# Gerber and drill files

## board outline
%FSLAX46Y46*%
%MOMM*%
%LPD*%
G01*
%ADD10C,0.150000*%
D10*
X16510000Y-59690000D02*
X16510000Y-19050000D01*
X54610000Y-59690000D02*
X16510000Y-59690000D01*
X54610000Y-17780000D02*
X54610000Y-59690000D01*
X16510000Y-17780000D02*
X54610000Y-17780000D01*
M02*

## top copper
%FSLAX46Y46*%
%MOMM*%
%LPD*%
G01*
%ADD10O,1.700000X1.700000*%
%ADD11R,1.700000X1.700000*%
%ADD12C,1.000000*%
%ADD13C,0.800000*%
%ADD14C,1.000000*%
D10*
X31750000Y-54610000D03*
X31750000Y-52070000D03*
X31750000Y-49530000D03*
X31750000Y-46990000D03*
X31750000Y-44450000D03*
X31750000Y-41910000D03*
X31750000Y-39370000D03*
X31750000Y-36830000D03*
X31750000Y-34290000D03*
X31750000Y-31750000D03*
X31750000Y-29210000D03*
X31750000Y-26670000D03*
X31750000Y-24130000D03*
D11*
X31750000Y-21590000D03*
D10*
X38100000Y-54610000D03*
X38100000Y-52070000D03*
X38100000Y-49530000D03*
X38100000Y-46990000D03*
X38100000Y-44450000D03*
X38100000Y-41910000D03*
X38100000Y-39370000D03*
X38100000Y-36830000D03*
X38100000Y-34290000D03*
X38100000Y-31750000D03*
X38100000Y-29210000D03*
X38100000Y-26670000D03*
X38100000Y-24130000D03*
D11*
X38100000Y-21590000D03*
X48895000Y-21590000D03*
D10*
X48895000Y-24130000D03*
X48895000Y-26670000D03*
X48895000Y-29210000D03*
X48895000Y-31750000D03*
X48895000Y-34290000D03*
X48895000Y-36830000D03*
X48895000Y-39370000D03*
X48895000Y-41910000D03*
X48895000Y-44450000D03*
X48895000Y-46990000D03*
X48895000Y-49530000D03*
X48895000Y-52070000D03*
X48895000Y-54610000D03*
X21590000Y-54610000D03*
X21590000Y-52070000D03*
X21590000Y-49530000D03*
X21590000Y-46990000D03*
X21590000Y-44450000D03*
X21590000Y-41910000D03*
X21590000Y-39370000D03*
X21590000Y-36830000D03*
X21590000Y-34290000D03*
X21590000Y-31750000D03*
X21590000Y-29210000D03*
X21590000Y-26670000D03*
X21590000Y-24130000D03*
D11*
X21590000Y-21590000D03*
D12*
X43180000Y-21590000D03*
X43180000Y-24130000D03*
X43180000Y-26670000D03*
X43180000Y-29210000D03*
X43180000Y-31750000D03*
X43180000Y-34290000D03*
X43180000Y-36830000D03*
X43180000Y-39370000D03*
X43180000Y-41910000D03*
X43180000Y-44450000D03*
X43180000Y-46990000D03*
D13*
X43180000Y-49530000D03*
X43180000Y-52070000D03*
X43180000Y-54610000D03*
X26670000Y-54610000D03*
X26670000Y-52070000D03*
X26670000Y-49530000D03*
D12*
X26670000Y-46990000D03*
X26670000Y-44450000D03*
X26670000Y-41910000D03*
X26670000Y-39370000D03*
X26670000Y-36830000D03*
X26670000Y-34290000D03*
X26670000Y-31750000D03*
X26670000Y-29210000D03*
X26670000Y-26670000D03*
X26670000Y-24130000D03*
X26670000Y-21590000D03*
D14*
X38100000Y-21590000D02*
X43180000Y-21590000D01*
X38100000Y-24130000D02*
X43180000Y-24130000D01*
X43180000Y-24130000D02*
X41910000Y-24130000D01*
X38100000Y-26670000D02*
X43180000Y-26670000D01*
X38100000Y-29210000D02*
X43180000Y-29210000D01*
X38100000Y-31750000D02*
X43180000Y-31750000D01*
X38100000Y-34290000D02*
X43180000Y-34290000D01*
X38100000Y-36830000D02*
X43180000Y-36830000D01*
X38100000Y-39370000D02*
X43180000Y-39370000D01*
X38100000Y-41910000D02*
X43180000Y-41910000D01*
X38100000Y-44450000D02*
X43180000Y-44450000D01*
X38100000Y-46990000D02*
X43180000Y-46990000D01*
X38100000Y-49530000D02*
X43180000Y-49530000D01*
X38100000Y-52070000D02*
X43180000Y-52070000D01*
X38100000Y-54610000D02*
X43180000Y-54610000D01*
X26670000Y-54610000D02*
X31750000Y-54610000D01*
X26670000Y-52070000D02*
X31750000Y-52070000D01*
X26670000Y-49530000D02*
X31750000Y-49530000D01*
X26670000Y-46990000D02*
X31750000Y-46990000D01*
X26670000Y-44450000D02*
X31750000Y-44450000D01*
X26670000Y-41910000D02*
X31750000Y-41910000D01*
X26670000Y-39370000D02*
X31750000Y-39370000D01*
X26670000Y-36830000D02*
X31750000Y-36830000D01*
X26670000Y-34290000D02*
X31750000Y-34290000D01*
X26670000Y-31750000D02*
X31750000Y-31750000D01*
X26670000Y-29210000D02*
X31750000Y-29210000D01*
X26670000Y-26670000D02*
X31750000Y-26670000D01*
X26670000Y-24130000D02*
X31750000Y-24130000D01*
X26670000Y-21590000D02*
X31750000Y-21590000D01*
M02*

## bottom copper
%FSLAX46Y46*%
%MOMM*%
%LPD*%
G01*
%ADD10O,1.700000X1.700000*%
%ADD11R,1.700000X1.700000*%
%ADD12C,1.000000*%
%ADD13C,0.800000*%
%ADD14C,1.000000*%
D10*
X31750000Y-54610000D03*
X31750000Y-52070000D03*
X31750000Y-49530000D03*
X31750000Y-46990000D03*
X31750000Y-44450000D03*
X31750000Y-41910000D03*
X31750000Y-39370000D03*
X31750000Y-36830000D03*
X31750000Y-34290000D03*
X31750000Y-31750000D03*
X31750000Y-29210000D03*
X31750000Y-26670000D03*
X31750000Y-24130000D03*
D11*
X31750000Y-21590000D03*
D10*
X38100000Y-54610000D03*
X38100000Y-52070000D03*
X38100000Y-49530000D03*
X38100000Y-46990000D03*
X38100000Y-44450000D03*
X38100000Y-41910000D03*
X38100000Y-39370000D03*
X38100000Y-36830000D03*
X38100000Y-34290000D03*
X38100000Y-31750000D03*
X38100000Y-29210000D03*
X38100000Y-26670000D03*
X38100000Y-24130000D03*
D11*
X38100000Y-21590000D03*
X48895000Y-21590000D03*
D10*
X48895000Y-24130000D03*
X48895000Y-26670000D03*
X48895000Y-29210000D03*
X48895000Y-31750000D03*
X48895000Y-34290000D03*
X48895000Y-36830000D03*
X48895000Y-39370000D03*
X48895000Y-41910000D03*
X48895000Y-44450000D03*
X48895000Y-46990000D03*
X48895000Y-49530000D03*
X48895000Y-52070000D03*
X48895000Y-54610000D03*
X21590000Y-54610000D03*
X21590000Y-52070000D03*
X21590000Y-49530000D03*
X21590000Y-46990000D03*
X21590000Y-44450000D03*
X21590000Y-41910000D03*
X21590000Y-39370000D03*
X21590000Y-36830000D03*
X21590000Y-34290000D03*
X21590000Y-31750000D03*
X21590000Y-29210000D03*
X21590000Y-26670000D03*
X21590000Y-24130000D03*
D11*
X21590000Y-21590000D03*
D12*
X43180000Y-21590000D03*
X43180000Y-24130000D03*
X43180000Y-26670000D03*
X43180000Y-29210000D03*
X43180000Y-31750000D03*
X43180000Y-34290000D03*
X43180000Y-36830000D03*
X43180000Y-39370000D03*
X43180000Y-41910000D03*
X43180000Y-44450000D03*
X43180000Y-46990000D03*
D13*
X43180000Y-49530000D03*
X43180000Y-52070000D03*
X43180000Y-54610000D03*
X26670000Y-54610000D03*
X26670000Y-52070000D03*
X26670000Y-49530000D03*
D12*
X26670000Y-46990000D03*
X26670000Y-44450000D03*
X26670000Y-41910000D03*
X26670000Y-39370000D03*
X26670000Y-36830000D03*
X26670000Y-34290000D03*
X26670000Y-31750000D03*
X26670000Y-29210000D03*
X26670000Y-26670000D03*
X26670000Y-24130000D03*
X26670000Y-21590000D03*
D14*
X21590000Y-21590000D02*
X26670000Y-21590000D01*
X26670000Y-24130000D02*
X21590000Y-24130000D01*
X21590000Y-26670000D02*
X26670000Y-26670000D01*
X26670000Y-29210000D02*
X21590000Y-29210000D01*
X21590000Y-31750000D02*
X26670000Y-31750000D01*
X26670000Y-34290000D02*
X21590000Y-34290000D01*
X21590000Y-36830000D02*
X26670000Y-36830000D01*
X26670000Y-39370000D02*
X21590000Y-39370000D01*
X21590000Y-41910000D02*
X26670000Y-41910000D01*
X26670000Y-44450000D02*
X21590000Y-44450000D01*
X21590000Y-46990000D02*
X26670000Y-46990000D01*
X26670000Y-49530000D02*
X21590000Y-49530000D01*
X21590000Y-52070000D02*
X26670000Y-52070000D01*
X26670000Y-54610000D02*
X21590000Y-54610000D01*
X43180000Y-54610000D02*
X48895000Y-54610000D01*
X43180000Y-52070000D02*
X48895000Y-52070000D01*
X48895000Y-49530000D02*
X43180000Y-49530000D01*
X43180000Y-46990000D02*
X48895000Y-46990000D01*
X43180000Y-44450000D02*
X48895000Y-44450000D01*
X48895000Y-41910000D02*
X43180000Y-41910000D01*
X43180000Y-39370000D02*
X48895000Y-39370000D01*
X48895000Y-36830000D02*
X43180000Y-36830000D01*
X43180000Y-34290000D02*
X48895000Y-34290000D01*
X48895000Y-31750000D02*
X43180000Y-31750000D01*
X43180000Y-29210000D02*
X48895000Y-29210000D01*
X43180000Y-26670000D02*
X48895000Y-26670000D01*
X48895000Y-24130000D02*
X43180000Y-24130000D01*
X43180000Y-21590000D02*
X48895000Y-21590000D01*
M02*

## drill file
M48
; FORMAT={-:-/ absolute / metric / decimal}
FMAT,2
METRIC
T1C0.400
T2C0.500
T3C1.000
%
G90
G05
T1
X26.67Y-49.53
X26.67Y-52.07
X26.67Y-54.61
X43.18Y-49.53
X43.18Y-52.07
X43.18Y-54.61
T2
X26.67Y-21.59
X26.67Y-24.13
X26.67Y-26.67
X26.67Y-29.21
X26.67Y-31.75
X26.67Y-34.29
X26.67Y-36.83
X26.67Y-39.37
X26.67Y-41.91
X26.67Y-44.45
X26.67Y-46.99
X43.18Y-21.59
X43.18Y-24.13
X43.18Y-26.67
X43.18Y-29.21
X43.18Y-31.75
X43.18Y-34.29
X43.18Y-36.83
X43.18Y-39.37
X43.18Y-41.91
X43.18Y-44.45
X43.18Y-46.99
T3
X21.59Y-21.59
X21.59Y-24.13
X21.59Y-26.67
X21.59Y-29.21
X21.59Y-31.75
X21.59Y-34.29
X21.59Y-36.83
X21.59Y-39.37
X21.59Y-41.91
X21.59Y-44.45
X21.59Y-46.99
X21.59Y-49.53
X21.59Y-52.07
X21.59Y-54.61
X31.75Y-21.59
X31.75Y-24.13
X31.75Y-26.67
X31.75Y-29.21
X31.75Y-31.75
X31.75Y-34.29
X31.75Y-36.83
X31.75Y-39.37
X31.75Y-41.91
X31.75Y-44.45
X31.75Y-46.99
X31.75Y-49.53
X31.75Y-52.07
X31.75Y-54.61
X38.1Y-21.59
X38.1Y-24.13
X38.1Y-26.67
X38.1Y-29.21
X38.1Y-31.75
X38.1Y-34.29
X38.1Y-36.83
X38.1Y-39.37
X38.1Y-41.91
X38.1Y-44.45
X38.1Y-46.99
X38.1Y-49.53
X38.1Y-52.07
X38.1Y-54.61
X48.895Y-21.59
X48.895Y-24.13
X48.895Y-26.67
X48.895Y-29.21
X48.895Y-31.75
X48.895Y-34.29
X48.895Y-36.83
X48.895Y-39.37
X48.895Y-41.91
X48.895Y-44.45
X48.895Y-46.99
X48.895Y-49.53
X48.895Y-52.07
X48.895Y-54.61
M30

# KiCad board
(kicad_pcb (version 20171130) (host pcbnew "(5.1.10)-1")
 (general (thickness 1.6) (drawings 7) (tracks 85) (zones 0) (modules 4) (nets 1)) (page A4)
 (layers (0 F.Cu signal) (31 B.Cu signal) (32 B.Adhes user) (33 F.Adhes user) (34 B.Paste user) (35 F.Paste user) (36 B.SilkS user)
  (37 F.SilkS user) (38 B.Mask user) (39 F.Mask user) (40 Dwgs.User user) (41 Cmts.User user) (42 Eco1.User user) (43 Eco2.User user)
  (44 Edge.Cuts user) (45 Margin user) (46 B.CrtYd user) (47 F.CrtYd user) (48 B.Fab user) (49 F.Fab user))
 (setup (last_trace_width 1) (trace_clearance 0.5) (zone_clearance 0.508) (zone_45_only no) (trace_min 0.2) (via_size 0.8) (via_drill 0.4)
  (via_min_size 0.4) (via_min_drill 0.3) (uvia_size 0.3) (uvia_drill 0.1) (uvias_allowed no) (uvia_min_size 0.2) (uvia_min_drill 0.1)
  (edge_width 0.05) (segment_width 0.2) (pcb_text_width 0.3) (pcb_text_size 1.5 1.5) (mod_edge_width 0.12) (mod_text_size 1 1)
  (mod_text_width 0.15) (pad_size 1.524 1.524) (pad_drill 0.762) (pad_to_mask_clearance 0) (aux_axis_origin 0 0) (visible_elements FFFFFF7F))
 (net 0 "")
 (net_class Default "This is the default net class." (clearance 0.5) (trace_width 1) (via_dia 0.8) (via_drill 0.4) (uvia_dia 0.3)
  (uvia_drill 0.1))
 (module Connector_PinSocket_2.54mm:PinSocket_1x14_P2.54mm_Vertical (layer F.Cu) (at 31.75 21.59)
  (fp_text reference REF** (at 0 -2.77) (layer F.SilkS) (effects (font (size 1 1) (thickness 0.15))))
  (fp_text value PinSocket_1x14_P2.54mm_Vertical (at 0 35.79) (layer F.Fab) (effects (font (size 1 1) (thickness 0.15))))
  (pad 14 thru_hole oval (at 0 33.02) (size 1.7 1.7) (drill 1) (layers *.Cu *.Mask))
  (pad 13 thru_hole oval (at 0 30.48) (size 1.7 1.7) (drill 1) (layers *.Cu *.Mask))
  (pad 12 thru_hole oval (at 0 27.94) (size 1.7 1.7) (drill 1) (layers *.Cu *.Mask))
  (pad 11 thru_hole oval (at 0 25.4) (size 1.7 1.7) (drill 1) (layers *.Cu *.Mask))
  (pad 10 thru_hole oval (at 0 22.86) (size 1.7 1.7) (drill 1) (layers *.Cu *.Mask))
  (pad 9 thru_hole oval (at 0 20.32) (size 1.7 1.7) (drill 1) (layers *.Cu *.Mask))
  (pad 8 thru_hole oval (at 0 17.78) (size 1.7 1.7) (drill 1) (layers *.Cu *.Mask))
  (pad 7 thru_hole oval (at 0 15.24) (size 1.7 1.7) (drill 1) (layers *.Cu *.Mask))
  (pad 6 thru_hole oval (at 0 12.7) (size 1.7 1.7) (drill 1) (layers *.Cu *.Mask))
  (pad 5 thru_hole oval (at 0 10.16) (size 1.7 1.7) (drill 1) (layers *.Cu *.Mask))
  (pad 4 thru_hole oval (at 0 7.62) (size 1.7 1.7) (drill 1) (layers *.Cu *.Mask))
  (pad 3 thru_hole oval (at 0 5.08) (size 1.7 1.7) (drill 1) (layers *.Cu *.Mask))
  (pad 2 thru_hole oval (at 0 2.54) (size 1.7 1.7) (drill 1) (layers *.Cu *.Mask))
  (pad 1 thru_hole rect (at 0 0) (size 1.7 1.7) (drill 1) (layers *.Cu *.Mask)))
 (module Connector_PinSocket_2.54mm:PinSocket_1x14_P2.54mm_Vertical (layer F.Cu) (at 38.1 21.59)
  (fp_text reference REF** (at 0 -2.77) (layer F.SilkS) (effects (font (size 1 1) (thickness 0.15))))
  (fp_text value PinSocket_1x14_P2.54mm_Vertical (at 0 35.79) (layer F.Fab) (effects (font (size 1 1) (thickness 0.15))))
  (pad 14 thru_hole oval (at 0 33.02) (size 1.7 1.7) (drill 1) (layers *.Cu *.Mask))
  (pad 13 thru_hole oval (at 0 30.48) (size 1.7 1.7) (drill 1) (layers *.Cu *.Mask))
  (pad 12 thru_hole oval (at 0 27.94) (size 1.7 1.7) (drill 1) (layers *.Cu *.Mask))
  (pad 11 thru_hole oval (at 0 25.4) (size 1.7 1.7) (drill 1) (layers *.Cu *.Mask))
  (pad 10 thru_hole oval (at 0 22.86) (size 1.7 1.7) (drill 1) (layers *.Cu *.Mask))
  (pad 9 thru_hole oval (at 0 20.32) (size 1.7 1.7) (drill 1) (layers *.Cu *.Mask))
  (pad 8 thru_hole oval (at 0 17.78) (size 1.7 1.7) (drill 1) (layers *.Cu *.Mask))
  (pad 7 thru_hole oval (at 0 15.24) (size 1.7 1.7) (drill 1) (layers *.Cu *.Mask))
  (pad 6 thru_hole oval (at 0 12.7) (size 1.7 1.7) (drill 1) (layers *.Cu *.Mask))
  (pad 5 thru_hole oval (at 0 10.16) (size 1.7 1.7) (drill 1) (layers *.Cu *.Mask))
  (pad 4 thru_hole oval (at 0 7.62) (size 1.7 1.7) (drill 1) (layers *.Cu *.Mask))
  (pad 3 thru_hole oval (at 0 5.08) (size 1.7 1.7) (drill 1) (layers *.Cu *.Mask))
  (pad 2 thru_hole oval (at 0 2.54) (size 1.7 1.7) (drill 1) (layers *.Cu *.Mask))
  (pad 1 thru_hole rect (at 0 0) (size 1.7 1.7) (drill 1) (layers *.Cu *.Mask)))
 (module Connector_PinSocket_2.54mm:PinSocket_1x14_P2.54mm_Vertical (layer F.Cu) (at 48.895 21.59)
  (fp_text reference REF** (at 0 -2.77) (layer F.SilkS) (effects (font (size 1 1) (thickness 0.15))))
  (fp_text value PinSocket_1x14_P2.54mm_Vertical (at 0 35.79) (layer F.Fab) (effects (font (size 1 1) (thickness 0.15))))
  (pad 1 thru_hole rect (at 0 0) (size 1.7 1.7) (drill 1) (layers *.Cu *.Mask))
  (pad 2 thru_hole oval (at 0 2.54) (size 1.7 1.7) (drill 1) (layers *.Cu *.Mask))
  (pad 3 thru_hole oval (at 0 5.08) (size 1.7 1.7) (drill 1) (layers *.Cu *.Mask))
  (pad 4 thru_hole oval (at 0 7.62) (size 1.7 1.7) (drill 1) (layers *.Cu *.Mask))
  (pad 5 thru_hole oval (at 0 10.16) (size 1.7 1.7) (drill 1) (layers *.Cu *.Mask))
  (pad 6 thru_hole oval (at 0 12.7) (size 1.7 1.7) (drill 1) (layers *.Cu *.Mask))
  (pad 7 thru_hole oval (at 0 15.24) (size 1.7 1.7) (drill 1) (layers *.Cu *.Mask))
  (pad 8 thru_hole oval (at 0 17.78) (size 1.7 1.7) (drill 1) (layers *.Cu *.Mask))
  (pad 9 thru_hole oval (at 0 20.32) (size 1.7 1.7) (drill 1) (layers *.Cu *.Mask))
  (pad 10 thru_hole oval (at 0 22.86) (size 1.7 1.7) (drill 1) (layers *.Cu *.Mask))
  (pad 11 thru_hole oval (at 0 25.4) (size 1.7 1.7) (drill 1) (layers *.Cu *.Mask))
  (pad 12 thru_hole oval (at 0 27.94) (size 1.7 1.7) (drill 1) (layers *.Cu *.Mask))
  (pad 13 thru_hole oval (at 0 30.48) (size 1.7 1.7) (drill 1) (layers *.Cu *.Mask))
  (pad 14 thru_hole oval (at 0 33.02) (size 1.7 1.7) (drill 1) (layers *.Cu *.Mask)))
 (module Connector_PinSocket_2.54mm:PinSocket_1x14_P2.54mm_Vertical (layer F.Cu) (at 21.59 21.59)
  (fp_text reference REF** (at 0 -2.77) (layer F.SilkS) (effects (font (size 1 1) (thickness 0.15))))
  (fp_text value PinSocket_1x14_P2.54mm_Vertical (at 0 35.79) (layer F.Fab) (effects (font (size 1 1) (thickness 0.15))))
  (pad 14 thru_hole oval (at 0 33.02) (size 1.7 1.7) (drill 1) (layers *.Cu *.Mask))
  (pad 13 thru_hole oval (at 0 30.48) (size 1.7 1.7) (drill 1) (layers *.Cu *.Mask))
  (pad 12 thru_hole oval (at 0 27.94) (size 1.7 1.7) (drill 1) (layers *.Cu *.Mask))
  (pad 11 thru_hole oval (at 0 25.4) (size 1.7 1.7) (drill 1) (layers *.Cu *.Mask))
  (pad 10 thru_hole oval (at 0 22.86) (size 1.7 1.7) (drill 1) (layers *.Cu *.Mask))
  (pad 9 thru_hole oval (at 0 20.32) (size 1.7 1.7) (drill 1) (layers *.Cu *.Mask))
  (pad 8 thru_hole oval (at 0 17.78) (size 1.7 1.7) (drill 1) (layers *.Cu *.Mask))
  (pad 7 thru_hole oval (at 0 15.24) (size 1.7 1.7) (drill 1) (layers *.Cu *.Mask))
  (pad 6 thru_hole oval (at 0 12.7) (size 1.7 1.7) (drill 1) (layers *.Cu *.Mask))
  (pad 5 thru_hole oval (at 0 10.16) (size 1.7 1.7) (drill 1) (layers *.Cu *.Mask))
  (pad 4 thru_hole oval (at 0 7.62) (size 1.7 1.7) (drill 1) (layers *.Cu *.Mask))
  (pad 3 thru_hole oval (at 0 5.08) (size 1.7 1.7) (drill 1) (layers *.Cu *.Mask))
  (pad 2 thru_hole oval (at 0 2.54) (size 1.7 1.7) (drill 1) (layers *.Cu *.Mask))
  (pad 1 thru_hole rect (at 0 0) (size 1.7 1.7) (drill 1) (layers *.Cu *.Mask)))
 (gr_line (start 16.51 59.69) (end 16.51 19.05) (layer Edge.Cuts) (width 0.15))
 (gr_line (start 54.61 59.69) (end 16.51 59.69) (layer Edge.Cuts) (width 0.15))
 (gr_line (start 54.61 17.78) (end 54.61 59.69) (layer Edge.Cuts) (width 0.15))
 (gr_line (start 16.51 17.78) (end 54.61 17.78) (layer Edge.Cuts) (width 0.15))
 (via (at 43.18 21.59) (size 1) (drill 0.5) (layers F.Cu B.Cu) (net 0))
 (via (at 43.18 24.13) (size 1) (drill 0.5) (layers F.Cu B.Cu) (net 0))
 (via (at 43.18 26.67) (size 1) (drill 0.5) (layers F.Cu B.Cu) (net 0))
 (via (at 43.18 29.21) (size 1) (drill 0.5) (layers F.Cu B.Cu) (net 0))
 (via (at 43.18 31.75) (size 1) (drill 0.5) (layers F.Cu B.Cu) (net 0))
 (via (at 43.18 34.29) (size 1) (drill 0.5) (layers F.Cu B.Cu) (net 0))
 (via (at 43.18 36.83) (size 1) (drill 0.5) (layers F.Cu B.Cu) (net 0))
 (via (at 43.18 39.37) (size 1) (drill 0.5) (layers F.Cu B.Cu) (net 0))
 (via (at 43.18 41.91) (size 1) (drill 0.5) (layers F.Cu B.Cu) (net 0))
 (via (at 43.18 44.45) (size 1) (drill 0.5) (layers F.Cu B.Cu) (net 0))
 (via (at 43.18 46.99) (size 1) (drill 0.5) (layers F.Cu B.Cu) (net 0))
 (via (at 43.18 49.53) (size 0.8) (drill 0.4) (layers F.Cu B.Cu) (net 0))
 (via (at 43.18 52.07) (size 0.8) (drill 0.4) (layers F.Cu B.Cu) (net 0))
 (via (at 43.18 54.61) (size 0.8) (drill 0.4) (layers F.Cu B.Cu) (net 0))
 (via (at 26.67 54.61) (size 0.8) (drill 0.4) (layers F.Cu B.Cu) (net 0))
 (via (at 26.67 52.07) (size 0.8) (drill 0.4) (layers F.Cu B.Cu) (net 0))
 (via (at 26.67 49.53) (size 0.8) (drill 0.4) (layers F.Cu B.Cu) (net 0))
 (via (at 26.67 46.99) (size 1) (drill 0.5) (layers F.Cu B.Cu) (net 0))
 (via (at 26.67 44.45) (size 1) (drill 0.5) (layers F.Cu B.Cu) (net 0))
 (via (at 26.67 41.91) (size 1) (drill 0.5) (layers F.Cu B.Cu) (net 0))
 (via (at 26.67 39.37) (size 1) (drill 0.5) (layers F.Cu B.Cu) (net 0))
 (via (at 26.67 36.83) (size 1) (drill 0.5) (layers F.Cu B.Cu) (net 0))
 (via (at 26.67 34.29) (size 1) (drill 0.5) (layers F.Cu B.Cu) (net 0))
 (via (at 26.67 31.75) (size 1) (drill 0.5) (layers F.Cu B.Cu) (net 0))
 (via (at 26.67 29.21) (size 1) (drill 0.5) (layers F.Cu B.Cu) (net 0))
 (via (at 26.67 26.67) (size 1) (drill 0.5) (layers F.Cu B.Cu) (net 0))
 (via (at 26.67 24.13) (size 1) (drill 0.5) (layers F.Cu B.Cu) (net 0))
 (via (at 26.67 21.59) (size 1) (drill 0.5) (layers F.Cu B.Cu) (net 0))
 (segment (start 38.1 21.59) (end 43.18 21.59) (width 1) (layer F.Cu) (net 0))
 (segment (start 38.1 24.13) (end 43.18 24.13) (width 1) (layer F.Cu) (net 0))
 (segment (start 43.18 24.13) (end 41.91 24.13) (width 1) (layer F.Cu) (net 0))
 (segment (start 38.1 26.67) (end 43.18 26.67) (width 1) (layer F.Cu) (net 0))
 (segment (start 38.1 29.21) (end 43.18 29.21) (width 1) (layer F.Cu) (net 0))
 (segment (start 38.1 31.75) (end 43.18 31.75) (width 1) (layer F.Cu) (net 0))
 (segment (start 38.1 34.29) (end 43.18 34.29) (width 1) (layer F.Cu) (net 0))
 (segment (start 38.1 36.83) (end 43.18 36.83) (width 1) (layer F.Cu) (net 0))
 (segment (start 38.1 39.37) (end 43.18 39.37) (width 1) (layer F.Cu) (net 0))
 (segment (start 38.1 41.91) (end 43.18 41.91) (width 1) (layer F.Cu) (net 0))
 (segment (start 38.1 44.45) (end 43.18 44.45) (width 1) (layer F.Cu) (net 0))
 (segment (start 38.1 46.99) (end 43.18 46.99) (width 1) (layer F.Cu) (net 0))
 (segment (start 38.1 49.53) (end 43.18 49.53) (width 1) (layer F.Cu) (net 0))
 (segment (start 38.1 52.07) (end 43.18 52.07) (width 1) (layer F.Cu) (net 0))
 (segment (start 38.1 54.61) (end 43.18 54.61) (width 1) (layer F.Cu) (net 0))
 (segment (start 26.67 54.61) (end 31.75 54.61) (width 1) (layer F.Cu) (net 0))
 (segment (start 26.67 52.07) (end 31.75 52.07) (width 1) (layer F.Cu) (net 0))
 (segment (start 26.67 49.53) (end 31.75 49.53) (width 1) (layer F.Cu) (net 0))
 (segment (start 26.67 46.99) (end 31.75 46.99) (width 1) (layer F.Cu) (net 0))
 (segment (start 26.67 44.45) (end 31.75 44.45) (width 1) (layer F.Cu) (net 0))
 (segment (start 26.67 41.91) (end 31.75 41.91) (width 1) (layer F.Cu) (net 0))
 (segment (start 26.67 39.37) (end 31.75 39.37) (width 1) (layer F.Cu) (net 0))
 (segment (start 26.67 36.83) (end 31.75 36.83) (width 1) (layer F.Cu) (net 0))
 (segment (start 26.67 34.29) (end 31.75 34.29) (width 1) (layer F.Cu) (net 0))
 (segment (start 26.67 31.75) (end 31.75 31.75) (width 1) (layer F.Cu) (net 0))
 (segment (start 26.67 29.21) (end 31.75 29.21) (width 1) (layer F.Cu) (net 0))
 (segment (start 26.67 26.67) (end 31.75 26.67) (width 1) (layer F.Cu) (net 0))
 (segment (start 26.67 24.13) (end 31.75 24.13) (width 1) (layer F.Cu) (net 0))
 (segment (start 26.67 21.59) (end 31.75 21.59) (width 1) (layer F.Cu) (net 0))
 (segment (start 21.59 21.59) (end 26.67 21.59) (width 1) (layer B.Cu) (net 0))
 (segment (start 26.67 24.13) (end 21.59 24.13) (width 1) (layer B.Cu) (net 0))
 (segment (start 21.59 26.67) (end 26.67 26.67) (width 1) (layer B.Cu) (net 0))
 (segment (start 26.67 29.21) (end 21.59 29.21) (width 1) (layer B.Cu) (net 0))
 (segment (start 21.59 31.75) (end 26.67 31.75) (width 1) (layer B.Cu) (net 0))
 (segment (start 26.67 34.29) (end 21.59 34.29) (width 1) (layer B.Cu) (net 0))
 (segment (start 21.59 36.83) (end 26.67 36.83) (width 1) (layer B.Cu) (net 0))
 (segment (start 26.67 39.37) (end 21.59 39.37) (width 1) (layer B.Cu) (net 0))
 (segment (start 21.59 41.91) (end 26.67 41.91) (width 1) (layer B.Cu) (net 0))
 (segment (start 26.67 44.45) (end 21.59 44.45) (width 1) (layer B.Cu) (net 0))
 (segment (start 21.59 46.99) (end 26.67 46.99) (width 1) (layer B.Cu) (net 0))
 (segment (start 26.67 49.53) (end 21.59 49.53) (width 1) (layer B.Cu) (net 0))
 (segment (start 21.59 52.07) (end 26.67 52.07) (width 1) (layer B.Cu) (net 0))
 (segment (start 26.67 54.61) (end 21.59 54.61) (width 1) (layer B.Cu) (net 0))
 (segment (start 43.18 54.61) (end 48.895 54.61) (width 1) (layer B.Cu) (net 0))
 (segment (start 43.18 52.07) (end 48.895 52.07) (width 1) (layer B.Cu) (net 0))
 (segment (start 48.895 49.53) (end 43.18 49.53) (width 1) (layer B.Cu) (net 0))
 (segment (start 43.18 46.99) (end 48.895 46.99) (width 1) (layer B.Cu) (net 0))
 (segment (start 43.18 44.45) (end 48.895 44.45) (width 1) (layer B.Cu) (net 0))
 (segment (start 48.895 41.91) (end 43.18 41.91) (width 1) (layer B.Cu) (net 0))
 (segment (start 43.18 39.37) (end 48.895 39.37) (width 1) (layer B.Cu) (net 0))
 (segment (start 48.895 36.83) (end 43.18 36.83) (width 1) (layer B.Cu) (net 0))
 (segment (start 43.18 34.29) (end 48.895 34.29) (width 1) (layer B.Cu) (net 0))
 (segment (start 48.895 31.75) (end 43.18 31.75) (width 1) (layer B.Cu) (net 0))
 (segment (start 43.18 29.21) (end 48.895 29.21) (width 1) (layer B.Cu) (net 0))
 (segment (start 43.18 26.67) (end 48.895 26.67) (width 1) (layer B.Cu) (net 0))
 (segment (start 48.895 24.13) (end 43.18 24.13) (width 1) (layer B.Cu) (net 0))
 (segment (start 43.18 21.59) (end 48.895 21.59) (width 1) (layer B.Cu) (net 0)))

